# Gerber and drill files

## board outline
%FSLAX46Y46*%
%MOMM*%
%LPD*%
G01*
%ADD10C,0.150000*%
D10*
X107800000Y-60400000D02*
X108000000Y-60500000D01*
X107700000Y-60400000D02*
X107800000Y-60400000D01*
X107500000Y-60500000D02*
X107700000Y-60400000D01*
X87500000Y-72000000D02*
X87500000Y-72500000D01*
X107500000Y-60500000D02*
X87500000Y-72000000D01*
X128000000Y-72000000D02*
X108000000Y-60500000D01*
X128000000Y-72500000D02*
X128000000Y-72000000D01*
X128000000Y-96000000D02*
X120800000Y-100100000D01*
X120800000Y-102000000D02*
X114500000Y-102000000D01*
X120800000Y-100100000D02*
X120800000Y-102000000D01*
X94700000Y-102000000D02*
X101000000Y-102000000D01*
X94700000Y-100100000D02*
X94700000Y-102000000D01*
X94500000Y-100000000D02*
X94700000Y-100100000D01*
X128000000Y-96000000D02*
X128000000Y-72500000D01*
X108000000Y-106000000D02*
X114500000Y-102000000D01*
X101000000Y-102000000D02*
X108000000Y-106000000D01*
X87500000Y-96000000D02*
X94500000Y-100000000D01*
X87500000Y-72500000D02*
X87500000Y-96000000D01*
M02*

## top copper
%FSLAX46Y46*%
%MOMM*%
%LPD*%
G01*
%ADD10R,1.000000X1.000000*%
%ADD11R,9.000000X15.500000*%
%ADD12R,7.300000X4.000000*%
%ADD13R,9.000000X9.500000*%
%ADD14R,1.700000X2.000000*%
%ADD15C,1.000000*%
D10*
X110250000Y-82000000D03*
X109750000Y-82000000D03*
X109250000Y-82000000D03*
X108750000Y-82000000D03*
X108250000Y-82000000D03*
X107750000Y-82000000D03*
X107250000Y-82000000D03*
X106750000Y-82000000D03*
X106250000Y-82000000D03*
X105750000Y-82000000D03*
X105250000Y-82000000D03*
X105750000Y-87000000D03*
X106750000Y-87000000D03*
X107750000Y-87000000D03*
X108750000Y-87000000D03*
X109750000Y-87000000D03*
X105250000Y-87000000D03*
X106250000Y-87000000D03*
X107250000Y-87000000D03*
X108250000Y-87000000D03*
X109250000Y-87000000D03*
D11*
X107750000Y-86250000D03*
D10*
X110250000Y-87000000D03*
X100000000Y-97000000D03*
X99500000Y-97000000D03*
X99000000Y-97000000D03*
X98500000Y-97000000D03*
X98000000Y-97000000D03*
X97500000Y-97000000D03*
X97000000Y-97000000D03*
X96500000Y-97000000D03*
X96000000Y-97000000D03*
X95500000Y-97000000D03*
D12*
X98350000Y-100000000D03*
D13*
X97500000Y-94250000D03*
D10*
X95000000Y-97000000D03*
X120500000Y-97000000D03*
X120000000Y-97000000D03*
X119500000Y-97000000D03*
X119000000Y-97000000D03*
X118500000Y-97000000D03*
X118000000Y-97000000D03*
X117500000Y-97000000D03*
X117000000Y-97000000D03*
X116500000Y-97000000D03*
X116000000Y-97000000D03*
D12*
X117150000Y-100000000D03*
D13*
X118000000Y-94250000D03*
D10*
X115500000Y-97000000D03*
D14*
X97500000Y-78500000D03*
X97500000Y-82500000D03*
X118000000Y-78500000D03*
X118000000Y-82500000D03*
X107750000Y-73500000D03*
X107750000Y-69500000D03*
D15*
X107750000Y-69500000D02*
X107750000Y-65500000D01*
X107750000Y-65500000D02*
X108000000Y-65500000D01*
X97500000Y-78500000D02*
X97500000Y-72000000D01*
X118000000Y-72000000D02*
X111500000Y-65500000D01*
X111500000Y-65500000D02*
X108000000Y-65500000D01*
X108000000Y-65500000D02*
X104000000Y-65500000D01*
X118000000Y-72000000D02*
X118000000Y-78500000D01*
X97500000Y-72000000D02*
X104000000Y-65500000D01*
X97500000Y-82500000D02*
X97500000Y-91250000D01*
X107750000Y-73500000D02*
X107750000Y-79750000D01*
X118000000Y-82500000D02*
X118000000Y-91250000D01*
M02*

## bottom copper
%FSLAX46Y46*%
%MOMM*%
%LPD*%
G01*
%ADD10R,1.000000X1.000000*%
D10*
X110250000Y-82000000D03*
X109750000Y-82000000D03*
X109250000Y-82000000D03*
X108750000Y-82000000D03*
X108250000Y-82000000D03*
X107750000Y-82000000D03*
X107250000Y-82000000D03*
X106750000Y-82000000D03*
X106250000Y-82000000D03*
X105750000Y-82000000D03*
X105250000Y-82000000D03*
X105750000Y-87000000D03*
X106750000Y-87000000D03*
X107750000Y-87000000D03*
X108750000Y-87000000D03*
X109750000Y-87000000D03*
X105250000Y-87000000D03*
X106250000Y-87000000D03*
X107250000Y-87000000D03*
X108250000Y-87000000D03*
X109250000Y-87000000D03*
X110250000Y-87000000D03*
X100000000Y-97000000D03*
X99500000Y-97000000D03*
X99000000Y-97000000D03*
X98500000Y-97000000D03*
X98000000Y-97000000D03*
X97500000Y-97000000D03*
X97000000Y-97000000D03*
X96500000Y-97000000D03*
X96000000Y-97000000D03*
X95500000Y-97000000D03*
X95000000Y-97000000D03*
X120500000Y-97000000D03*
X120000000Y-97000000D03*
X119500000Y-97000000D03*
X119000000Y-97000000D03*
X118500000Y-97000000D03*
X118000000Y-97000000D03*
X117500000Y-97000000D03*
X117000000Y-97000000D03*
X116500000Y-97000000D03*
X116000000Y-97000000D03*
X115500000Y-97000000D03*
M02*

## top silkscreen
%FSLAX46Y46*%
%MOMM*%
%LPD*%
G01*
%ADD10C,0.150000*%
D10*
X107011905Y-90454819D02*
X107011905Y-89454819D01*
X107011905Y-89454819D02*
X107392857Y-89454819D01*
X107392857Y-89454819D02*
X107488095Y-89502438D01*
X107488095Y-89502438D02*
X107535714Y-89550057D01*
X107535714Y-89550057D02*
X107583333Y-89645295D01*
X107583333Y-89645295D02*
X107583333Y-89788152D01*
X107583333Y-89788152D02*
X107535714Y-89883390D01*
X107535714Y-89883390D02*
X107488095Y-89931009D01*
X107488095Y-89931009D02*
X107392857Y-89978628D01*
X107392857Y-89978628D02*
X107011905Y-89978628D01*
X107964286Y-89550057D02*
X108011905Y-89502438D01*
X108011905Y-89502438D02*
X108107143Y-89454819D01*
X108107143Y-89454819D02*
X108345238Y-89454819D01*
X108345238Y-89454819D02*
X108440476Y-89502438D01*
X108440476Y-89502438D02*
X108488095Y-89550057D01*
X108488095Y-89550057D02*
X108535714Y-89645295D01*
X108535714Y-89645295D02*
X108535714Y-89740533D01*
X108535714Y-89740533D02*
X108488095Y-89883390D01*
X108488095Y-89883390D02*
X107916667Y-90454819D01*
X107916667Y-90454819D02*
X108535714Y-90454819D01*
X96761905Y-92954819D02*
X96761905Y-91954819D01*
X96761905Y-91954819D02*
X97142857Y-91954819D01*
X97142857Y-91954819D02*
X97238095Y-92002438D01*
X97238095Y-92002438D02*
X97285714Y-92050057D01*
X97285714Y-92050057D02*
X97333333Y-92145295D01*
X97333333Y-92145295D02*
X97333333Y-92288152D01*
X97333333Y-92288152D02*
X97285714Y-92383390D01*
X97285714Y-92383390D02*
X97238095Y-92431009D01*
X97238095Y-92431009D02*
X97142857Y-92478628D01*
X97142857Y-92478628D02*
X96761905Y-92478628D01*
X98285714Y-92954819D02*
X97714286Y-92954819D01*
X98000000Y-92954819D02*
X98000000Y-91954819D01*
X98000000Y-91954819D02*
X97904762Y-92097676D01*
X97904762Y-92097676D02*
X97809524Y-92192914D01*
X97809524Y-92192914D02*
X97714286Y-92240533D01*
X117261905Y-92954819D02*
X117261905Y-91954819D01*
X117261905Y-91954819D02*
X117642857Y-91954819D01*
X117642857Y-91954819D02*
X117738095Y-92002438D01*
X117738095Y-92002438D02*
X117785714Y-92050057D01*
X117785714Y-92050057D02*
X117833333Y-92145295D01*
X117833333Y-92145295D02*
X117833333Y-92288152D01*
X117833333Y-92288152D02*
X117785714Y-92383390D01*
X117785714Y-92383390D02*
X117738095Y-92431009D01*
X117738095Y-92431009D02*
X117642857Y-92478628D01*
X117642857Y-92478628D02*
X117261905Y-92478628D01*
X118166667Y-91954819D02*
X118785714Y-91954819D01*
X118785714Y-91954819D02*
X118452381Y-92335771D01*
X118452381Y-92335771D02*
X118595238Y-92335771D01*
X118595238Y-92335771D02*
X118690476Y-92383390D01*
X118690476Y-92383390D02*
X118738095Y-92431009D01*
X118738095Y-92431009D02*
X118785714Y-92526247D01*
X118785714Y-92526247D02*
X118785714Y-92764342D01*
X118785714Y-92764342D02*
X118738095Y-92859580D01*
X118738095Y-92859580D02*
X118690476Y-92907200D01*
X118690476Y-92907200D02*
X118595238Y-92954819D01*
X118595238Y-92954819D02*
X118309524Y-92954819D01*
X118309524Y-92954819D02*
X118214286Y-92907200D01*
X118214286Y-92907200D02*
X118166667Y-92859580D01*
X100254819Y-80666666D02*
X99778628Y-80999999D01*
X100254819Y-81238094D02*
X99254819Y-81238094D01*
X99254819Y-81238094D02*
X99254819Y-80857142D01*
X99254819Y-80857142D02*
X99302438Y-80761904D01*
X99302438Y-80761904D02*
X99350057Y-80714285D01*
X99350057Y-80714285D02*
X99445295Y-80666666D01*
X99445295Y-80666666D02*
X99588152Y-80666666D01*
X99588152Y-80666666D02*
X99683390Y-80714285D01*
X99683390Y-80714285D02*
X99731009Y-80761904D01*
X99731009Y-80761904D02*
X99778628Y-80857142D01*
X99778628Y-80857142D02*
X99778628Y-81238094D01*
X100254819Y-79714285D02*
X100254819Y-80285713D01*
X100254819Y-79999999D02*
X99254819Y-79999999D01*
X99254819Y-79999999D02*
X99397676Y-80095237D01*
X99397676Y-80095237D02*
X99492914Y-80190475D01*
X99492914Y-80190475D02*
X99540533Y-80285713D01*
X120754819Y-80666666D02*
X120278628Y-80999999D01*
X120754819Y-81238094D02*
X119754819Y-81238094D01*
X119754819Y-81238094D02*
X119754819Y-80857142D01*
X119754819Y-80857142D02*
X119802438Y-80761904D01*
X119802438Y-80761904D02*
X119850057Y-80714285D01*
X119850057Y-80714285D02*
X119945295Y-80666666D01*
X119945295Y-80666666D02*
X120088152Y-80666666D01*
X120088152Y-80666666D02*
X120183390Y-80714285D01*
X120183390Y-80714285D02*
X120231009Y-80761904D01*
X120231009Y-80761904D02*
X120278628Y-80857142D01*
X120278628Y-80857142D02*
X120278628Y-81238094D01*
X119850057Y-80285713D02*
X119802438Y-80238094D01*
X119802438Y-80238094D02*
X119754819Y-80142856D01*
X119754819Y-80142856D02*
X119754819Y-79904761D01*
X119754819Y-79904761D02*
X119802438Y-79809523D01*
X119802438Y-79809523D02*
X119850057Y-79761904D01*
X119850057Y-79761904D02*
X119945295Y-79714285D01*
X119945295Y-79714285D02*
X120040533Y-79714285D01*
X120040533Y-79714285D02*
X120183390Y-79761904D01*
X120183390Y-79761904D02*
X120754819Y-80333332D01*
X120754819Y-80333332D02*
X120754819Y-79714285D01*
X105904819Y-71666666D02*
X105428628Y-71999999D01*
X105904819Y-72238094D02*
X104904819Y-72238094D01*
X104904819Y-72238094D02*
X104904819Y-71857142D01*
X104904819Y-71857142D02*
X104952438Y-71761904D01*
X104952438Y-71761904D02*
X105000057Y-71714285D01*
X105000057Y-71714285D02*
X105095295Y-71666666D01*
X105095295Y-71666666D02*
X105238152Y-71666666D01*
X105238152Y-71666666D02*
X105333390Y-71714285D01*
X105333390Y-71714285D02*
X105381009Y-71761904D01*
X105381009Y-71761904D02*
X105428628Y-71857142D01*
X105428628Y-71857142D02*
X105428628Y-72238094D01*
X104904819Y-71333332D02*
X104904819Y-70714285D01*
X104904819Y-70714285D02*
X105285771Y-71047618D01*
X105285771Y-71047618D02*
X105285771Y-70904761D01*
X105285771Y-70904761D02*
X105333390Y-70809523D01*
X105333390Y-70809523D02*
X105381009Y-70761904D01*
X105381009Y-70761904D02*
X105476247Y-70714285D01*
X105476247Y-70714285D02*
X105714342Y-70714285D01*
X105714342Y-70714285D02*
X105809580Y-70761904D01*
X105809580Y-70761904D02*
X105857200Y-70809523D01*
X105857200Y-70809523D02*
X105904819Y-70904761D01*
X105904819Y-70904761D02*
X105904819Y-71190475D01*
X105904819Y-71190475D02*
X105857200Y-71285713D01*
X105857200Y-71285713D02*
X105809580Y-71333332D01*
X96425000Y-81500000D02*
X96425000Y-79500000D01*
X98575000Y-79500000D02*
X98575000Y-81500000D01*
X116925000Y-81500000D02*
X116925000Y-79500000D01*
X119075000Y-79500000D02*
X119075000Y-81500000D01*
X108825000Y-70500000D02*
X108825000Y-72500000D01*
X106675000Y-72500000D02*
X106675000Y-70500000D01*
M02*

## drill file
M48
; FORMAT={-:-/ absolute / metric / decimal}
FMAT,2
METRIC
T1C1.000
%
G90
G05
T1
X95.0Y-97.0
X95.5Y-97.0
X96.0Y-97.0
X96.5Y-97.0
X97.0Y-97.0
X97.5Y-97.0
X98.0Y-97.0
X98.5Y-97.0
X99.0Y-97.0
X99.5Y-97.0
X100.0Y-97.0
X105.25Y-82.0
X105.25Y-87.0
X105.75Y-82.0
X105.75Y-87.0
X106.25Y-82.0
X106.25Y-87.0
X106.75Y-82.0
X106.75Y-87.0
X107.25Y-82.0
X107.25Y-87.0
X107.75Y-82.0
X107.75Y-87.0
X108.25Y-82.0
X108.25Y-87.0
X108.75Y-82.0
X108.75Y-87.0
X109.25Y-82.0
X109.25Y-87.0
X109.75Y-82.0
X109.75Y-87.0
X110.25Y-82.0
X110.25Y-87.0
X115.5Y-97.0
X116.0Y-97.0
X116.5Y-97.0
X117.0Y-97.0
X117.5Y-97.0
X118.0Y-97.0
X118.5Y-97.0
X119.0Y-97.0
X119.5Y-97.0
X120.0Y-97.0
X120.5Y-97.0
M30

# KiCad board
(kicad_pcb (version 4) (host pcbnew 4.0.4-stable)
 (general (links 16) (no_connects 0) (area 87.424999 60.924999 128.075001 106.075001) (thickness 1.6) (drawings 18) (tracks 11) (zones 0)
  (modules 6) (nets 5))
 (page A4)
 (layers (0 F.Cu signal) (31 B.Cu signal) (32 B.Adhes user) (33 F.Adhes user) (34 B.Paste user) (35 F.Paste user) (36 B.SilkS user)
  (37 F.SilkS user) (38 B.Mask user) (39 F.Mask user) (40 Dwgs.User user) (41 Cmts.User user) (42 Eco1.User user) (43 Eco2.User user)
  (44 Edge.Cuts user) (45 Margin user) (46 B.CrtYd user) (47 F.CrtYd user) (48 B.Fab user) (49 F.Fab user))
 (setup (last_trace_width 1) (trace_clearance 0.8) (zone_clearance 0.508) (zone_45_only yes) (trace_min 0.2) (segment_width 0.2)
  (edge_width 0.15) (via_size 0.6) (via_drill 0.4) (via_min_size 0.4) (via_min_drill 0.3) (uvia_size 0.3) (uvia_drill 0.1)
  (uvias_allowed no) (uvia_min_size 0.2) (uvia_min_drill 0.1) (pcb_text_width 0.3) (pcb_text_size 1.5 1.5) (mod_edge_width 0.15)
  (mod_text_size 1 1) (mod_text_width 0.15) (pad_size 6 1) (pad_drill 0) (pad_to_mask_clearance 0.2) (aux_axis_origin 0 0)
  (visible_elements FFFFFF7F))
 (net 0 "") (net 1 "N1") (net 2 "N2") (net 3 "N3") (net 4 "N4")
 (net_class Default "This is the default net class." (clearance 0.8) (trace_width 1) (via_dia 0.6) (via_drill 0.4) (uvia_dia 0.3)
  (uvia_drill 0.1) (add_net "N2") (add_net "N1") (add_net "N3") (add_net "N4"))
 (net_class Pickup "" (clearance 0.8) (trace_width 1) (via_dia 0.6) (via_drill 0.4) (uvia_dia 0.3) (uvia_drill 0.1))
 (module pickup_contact (layer F.Cu) (at 107.75 87 180)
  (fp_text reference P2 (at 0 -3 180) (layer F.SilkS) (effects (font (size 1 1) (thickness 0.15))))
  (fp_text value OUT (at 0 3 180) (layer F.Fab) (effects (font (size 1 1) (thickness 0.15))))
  (pad "" thru_hole rect (at -2.5 5 180) (size 1 1) (drill 1) (layers *.Cu *.Mask))
  (pad "" thru_hole rect (at -2 5 180) (size 1 1) (drill 1) (layers *.Cu *.Mask))
  (pad "" thru_hole rect (at -1.5 5 180) (size 1 1) (drill 1) (layers *.Cu *.Mask))
  (pad "" thru_hole rect (at -1 5 180) (size 1 1) (drill 1) (layers *.Cu *.Mask))
  (pad "" thru_hole rect (at -0.5 5 180) (size 1 1) (drill 1) (layers *.Cu *.Mask))
  (pad "" thru_hole rect (at 0 5 180) (size 1 1) (drill 1) (layers *.Cu *.Mask))
  (pad "" thru_hole rect (at 0.5 5 180) (size 1 1) (drill 1) (layers *.Cu *.Mask))
  (pad "" thru_hole rect (at 1 5 180) (size 1 1) (drill 1) (layers *.Cu *.Mask))
  (pad "" thru_hole rect (at 1.5 5 180) (size 1 1) (drill 1) (layers *.Cu *.Mask))
  (pad "" thru_hole rect (at 2 5 180) (size 1 1) (drill 1) (layers *.Cu *.Mask))
  (pad "" thru_hole rect (at 2.5 5 180) (size 1 1) (drill 1) (layers *.Cu *.Mask))
  (pad "" thru_hole rect (at 2 0 180) (size 1 1) (drill 1) (layers *.Cu *.Mask))
  (pad "" thru_hole rect (at 1 0 180) (size 1 1) (drill 1) (layers *.Cu *.Mask))
  (pad "" thru_hole rect (at 0 0 180) (size 1 1) (drill 1) (layers *.Cu *.Mask))
  (pad "" thru_hole rect (at -1 0 180) (size 1 1) (drill 1) (layers *.Cu *.Mask))
  (pad "" thru_hole rect (at -2 0 180) (size 1 1) (drill 1) (layers *.Cu *.Mask))
  (pad "" thru_hole rect (at 2.5 0 180) (size 1 1) (drill 1) (layers *.Cu *.Mask))
  (pad "" thru_hole rect (at 1.5 0 180) (size 1 1) (drill 1) (layers *.Cu *.Mask))
  (pad "" thru_hole rect (at 0.5 0 180) (size 1 1) (drill 1) (layers *.Cu *.Mask))
  (pad "" thru_hole rect (at -0.5 0 180) (size 1 1) (drill 1) (layers *.Cu *.Mask))
  (pad "" thru_hole rect (at -1.5 0 180) (size 1 1) (drill 1) (layers *.Cu *.Mask))
  (pad 1 smd rect (at 0 7.25 180) (size 9 15.5) (drill (offset 0 -6.5)) (layers F.Cu F.Paste F.Mask) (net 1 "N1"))
  (pad "" thru_hole rect (at -2.5 0 180) (size 1 1) (drill 1) (layers *.Cu *.Mask)))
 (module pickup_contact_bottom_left (layer F.Cu) (at 97.5 95.5)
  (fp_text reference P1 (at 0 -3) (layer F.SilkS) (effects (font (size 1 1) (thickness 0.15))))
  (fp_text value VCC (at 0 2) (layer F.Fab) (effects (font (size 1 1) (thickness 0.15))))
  (pad "" thru_hole rect (at 2.5 1.5) (size 1 1) (drill 1) (layers *.Cu *.Mask))
  (pad "" thru_hole rect (at 2 1.5) (size 1 1) (drill 1) (layers *.Cu *.Mask))
  (pad "" thru_hole rect (at 1.5 1.5) (size 1 1) (drill 1) (layers *.Cu *.Mask))
  (pad "" thru_hole rect (at 1 1.5) (size 1 1) (drill 1) (layers *.Cu *.Mask))
  (pad "" thru_hole rect (at 0.5 1.5) (size 1 1) (drill 1) (layers *.Cu *.Mask))
  (pad "" thru_hole rect (at 0 1.5) (size 1 1) (drill 1) (layers *.Cu *.Mask))
  (pad "" thru_hole rect (at -0.5 1.5) (size 1 1) (drill 1) (layers *.Cu *.Mask))
  (pad "" thru_hole rect (at -1 1.5) (size 1 1) (drill 1) (layers *.Cu *.Mask))
  (pad "" thru_hole rect (at -1.5 1.5) (size 1 1) (drill 1) (layers *.Cu *.Mask))
  (pad "" thru_hole rect (at -2 1.5) (size 1 1) (drill 1) (layers *.Cu *.Mask))
  (pad "" smd rect (at 0.85 4.5) (size 7.3 4) (layers F.Cu F.Paste F.Mask))
  (pad 1 smd rect (at 0 -4.25) (size 9 9.5) (drill (offset 0 3)) (layers F.Cu F.Paste F.Mask) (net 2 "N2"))
  (pad "" thru_hole rect (at -2.5 1.5) (size 1 1) (drill 1) (layers *.Cu *.Mask)))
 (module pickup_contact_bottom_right (layer F.Cu) (at 118 95.5)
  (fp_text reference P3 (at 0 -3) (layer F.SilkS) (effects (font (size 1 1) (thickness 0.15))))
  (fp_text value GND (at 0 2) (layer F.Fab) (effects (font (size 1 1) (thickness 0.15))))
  (pad 1 thru_hole rect (at 2.5 1.5) (size 1 1) (drill 1) (layers *.Cu *.Mask) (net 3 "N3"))
  (pad 1 thru_hole rect (at 2 1.5) (size 1 1) (drill 1) (layers *.Cu *.Mask) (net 3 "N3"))
  (pad 1 thru_hole rect (at 1.5 1.5) (size 1 1) (drill 1) (layers *.Cu *.Mask) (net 3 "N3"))
  (pad 1 thru_hole rect (at 1 1.5) (size 1 1) (drill 1) (layers *.Cu *.Mask) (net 3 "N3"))
  (pad 1 thru_hole rect (at 0.5 1.5) (size 1 1) (drill 1) (layers *.Cu *.Mask) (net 3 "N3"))
  (pad 1 thru_hole rect (at 0 1.5) (size 1 1) (drill 1) (layers *.Cu *.Mask) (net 3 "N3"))
  (pad 1 thru_hole rect (at -0.5 1.5) (size 1 1) (drill 1) (layers *.Cu *.Mask) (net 3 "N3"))
  (pad 1 thru_hole rect (at -1 1.5) (size 1 1) (drill 1) (layers *.Cu *.Mask) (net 3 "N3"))
  (pad 1 thru_hole rect (at -1.5 1.5) (size 1 1) (drill 1) (layers *.Cu *.Mask) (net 3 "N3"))
  (pad 1 thru_hole rect (at -2 1.5) (size 1 1) (drill 1) (layers *.Cu *.Mask) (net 3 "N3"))
  (pad "" smd rect (at -0.85 4.5) (size 7.3 4) (layers F.Cu F.Paste F.Mask))
  (pad 1 smd rect (at 0 -4.25) (size 9 9.5) (drill (offset 0 3)) (layers F.Cu F.Paste F.Mask) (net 3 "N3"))
  (pad 1 thru_hole rect (at -2.5 1.5) (size 1 1) (drill 1) (layers *.Cu *.Mask) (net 3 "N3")))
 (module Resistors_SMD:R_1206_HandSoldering (layer F.Cu) (at 97.5 80.5 270)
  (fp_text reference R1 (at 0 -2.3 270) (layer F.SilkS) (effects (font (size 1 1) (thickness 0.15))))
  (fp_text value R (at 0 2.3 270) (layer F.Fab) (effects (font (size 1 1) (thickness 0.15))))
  (fp_line (start 1 1.075) (end -1 1.075) (layer F.SilkS) (width 0.15))
  (fp_line (start -1 -1.075) (end 1 -1.075) (layer F.SilkS) (width 0.15))
  (pad 1 smd rect (at -2 0 270) (size 2 1.7) (layers F.Cu F.Paste F.Mask) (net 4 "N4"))
  (pad 2 smd rect (at 2 0 270) (size 2 1.7) (layers F.Cu F.Paste F.Mask) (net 2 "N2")))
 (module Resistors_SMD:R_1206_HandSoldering (layer F.Cu) (at 118 80.5 270)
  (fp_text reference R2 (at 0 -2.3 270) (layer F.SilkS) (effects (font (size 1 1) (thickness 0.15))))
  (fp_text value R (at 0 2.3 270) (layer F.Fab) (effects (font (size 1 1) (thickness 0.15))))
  (fp_line (start 1 1.075) (end -1 1.075) (layer F.SilkS) (width 0.15))
  (fp_line (start -1 -1.075) (end 1 -1.075) (layer F.SilkS) (width 0.15))
  (pad 1 smd rect (at -2 0 270) (size 2 1.7) (layers F.Cu F.Paste F.Mask) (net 4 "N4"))
  (pad 2 smd rect (at 2 0 270) (size 2 1.7) (layers F.Cu F.Paste F.Mask) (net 3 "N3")))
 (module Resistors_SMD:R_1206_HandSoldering (layer F.Cu) (at 107.75 71.5 90)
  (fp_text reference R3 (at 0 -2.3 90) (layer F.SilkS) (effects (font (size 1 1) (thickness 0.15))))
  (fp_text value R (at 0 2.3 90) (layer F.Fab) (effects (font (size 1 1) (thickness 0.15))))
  (fp_line (start 1 1.075) (end -1 1.075) (layer F.SilkS) (width 0.15))
  (fp_line (start -1 -1.075) (end 1 -1.075) (layer F.SilkS) (width 0.15))
  (pad 1 smd rect (at -2 0 90) (size 2 1.7) (layers F.Cu F.Paste F.Mask) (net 1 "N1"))
  (pad 2 smd rect (at 2 0 90) (size 2 1.7) (layers F.Cu F.Paste F.Mask) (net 4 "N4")))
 (gr_line (start 107.8 60.4) (end 108 60.5) (angle 90) (layer Edge.Cuts) (width 0.15))
 (gr_line (start 107.7 60.4) (end 107.8 60.4) (angle 90) (layer Edge.Cuts) (width 0.15))
 (gr_line (start 107.5 60.5) (end 107.7 60.4) (angle 90) (layer Edge.Cuts) (width 0.15))
 (gr_line (start 87.5 72) (end 87.5 72.5) (angle 90) (layer Edge.Cuts) (width 0.15))
 (gr_line (start 107.5 60.5) (end 87.5 72) (angle 90) (layer Edge.Cuts) (width 0.15))
 (gr_line (start 128 72) (end 108 60.5) (angle 90) (layer Edge.Cuts) (width 0.15))
 (gr_line (start 128 72.5) (end 128 72) (angle 90) (layer Edge.Cuts) (width 0.15))
 (gr_line (start 128 96) (end 120.8 100.1) (angle 90) (layer Edge.Cuts) (width 0.15))
 (gr_line (start 120.8 102) (end 114.5 102) (angle 90) (layer Edge.Cuts) (width 0.15))
 (gr_line (start 120.8 100.1) (end 120.8 102) (angle 90) (layer Edge.Cuts) (width 0.15))
 (gr_line (start 94.7 102) (end 101 102) (angle 90) (layer Edge.Cuts) (width 0.15))
 (gr_line (start 94.7 100.1) (end 94.7 102) (angle 90) (layer Edge.Cuts) (width 0.15))
 (gr_line (start 94.5 100) (end 94.7 100.1) (angle 90) (layer Edge.Cuts) (width 0.15))
 (gr_line (start 128 96) (end 128 72.5) (angle 90) (layer Edge.Cuts) (width 0.15))
 (gr_line (start 108 106) (end 114.5 102) (angle 90) (layer Edge.Cuts) (width 0.15))
 (gr_line (start 101 102) (end 108 106) (angle 90) (layer Edge.Cuts) (width 0.15))
 (gr_line (start 87.5 96) (end 94.5 100) (angle 90) (layer Edge.Cuts) (width 0.15))
 (gr_line (start 87.5 72.5) (end 87.5 96) (angle 90) (layer Edge.Cuts) (width 0.15))
 (segment (start 107.75 69.5) (end 107.75 65.5) (width 1) (layer F.Cu) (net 4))
 (segment (start 107.75 65.5) (end 108 65.5) (width 1) (layer F.Cu) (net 4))
 (segment (start 97.5 78.5) (end 97.5 72) (width 1) (layer F.Cu) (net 4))
 (segment (start 118 72) (end 111.5 65.5) (width 1) (layer F.Cu) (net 4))
 (segment (start 111.5 65.5) (end 108 65.5) (width 1) (layer F.Cu) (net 4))
 (segment (start 108 65.5) (end 104 65.5) (width 1) (layer F.Cu) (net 4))
 (segment (start 118 72) (end 118 78.5) (width 1) (layer F.Cu) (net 4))
 (segment (start 97.5 72) (end 104 65.5) (width 1) (layer F.Cu) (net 4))
 (segment (start 97.5 82.5) (end 97.5 91.25) (width 1) (layer F.Cu) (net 2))
 (segment (start 107.75 73.5) (end 107.75 79.75) (width 1) (layer F.Cu) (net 1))
 (segment (start 118 82.5) (end 118 91.25) (width 1) (layer F.Cu) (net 3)))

